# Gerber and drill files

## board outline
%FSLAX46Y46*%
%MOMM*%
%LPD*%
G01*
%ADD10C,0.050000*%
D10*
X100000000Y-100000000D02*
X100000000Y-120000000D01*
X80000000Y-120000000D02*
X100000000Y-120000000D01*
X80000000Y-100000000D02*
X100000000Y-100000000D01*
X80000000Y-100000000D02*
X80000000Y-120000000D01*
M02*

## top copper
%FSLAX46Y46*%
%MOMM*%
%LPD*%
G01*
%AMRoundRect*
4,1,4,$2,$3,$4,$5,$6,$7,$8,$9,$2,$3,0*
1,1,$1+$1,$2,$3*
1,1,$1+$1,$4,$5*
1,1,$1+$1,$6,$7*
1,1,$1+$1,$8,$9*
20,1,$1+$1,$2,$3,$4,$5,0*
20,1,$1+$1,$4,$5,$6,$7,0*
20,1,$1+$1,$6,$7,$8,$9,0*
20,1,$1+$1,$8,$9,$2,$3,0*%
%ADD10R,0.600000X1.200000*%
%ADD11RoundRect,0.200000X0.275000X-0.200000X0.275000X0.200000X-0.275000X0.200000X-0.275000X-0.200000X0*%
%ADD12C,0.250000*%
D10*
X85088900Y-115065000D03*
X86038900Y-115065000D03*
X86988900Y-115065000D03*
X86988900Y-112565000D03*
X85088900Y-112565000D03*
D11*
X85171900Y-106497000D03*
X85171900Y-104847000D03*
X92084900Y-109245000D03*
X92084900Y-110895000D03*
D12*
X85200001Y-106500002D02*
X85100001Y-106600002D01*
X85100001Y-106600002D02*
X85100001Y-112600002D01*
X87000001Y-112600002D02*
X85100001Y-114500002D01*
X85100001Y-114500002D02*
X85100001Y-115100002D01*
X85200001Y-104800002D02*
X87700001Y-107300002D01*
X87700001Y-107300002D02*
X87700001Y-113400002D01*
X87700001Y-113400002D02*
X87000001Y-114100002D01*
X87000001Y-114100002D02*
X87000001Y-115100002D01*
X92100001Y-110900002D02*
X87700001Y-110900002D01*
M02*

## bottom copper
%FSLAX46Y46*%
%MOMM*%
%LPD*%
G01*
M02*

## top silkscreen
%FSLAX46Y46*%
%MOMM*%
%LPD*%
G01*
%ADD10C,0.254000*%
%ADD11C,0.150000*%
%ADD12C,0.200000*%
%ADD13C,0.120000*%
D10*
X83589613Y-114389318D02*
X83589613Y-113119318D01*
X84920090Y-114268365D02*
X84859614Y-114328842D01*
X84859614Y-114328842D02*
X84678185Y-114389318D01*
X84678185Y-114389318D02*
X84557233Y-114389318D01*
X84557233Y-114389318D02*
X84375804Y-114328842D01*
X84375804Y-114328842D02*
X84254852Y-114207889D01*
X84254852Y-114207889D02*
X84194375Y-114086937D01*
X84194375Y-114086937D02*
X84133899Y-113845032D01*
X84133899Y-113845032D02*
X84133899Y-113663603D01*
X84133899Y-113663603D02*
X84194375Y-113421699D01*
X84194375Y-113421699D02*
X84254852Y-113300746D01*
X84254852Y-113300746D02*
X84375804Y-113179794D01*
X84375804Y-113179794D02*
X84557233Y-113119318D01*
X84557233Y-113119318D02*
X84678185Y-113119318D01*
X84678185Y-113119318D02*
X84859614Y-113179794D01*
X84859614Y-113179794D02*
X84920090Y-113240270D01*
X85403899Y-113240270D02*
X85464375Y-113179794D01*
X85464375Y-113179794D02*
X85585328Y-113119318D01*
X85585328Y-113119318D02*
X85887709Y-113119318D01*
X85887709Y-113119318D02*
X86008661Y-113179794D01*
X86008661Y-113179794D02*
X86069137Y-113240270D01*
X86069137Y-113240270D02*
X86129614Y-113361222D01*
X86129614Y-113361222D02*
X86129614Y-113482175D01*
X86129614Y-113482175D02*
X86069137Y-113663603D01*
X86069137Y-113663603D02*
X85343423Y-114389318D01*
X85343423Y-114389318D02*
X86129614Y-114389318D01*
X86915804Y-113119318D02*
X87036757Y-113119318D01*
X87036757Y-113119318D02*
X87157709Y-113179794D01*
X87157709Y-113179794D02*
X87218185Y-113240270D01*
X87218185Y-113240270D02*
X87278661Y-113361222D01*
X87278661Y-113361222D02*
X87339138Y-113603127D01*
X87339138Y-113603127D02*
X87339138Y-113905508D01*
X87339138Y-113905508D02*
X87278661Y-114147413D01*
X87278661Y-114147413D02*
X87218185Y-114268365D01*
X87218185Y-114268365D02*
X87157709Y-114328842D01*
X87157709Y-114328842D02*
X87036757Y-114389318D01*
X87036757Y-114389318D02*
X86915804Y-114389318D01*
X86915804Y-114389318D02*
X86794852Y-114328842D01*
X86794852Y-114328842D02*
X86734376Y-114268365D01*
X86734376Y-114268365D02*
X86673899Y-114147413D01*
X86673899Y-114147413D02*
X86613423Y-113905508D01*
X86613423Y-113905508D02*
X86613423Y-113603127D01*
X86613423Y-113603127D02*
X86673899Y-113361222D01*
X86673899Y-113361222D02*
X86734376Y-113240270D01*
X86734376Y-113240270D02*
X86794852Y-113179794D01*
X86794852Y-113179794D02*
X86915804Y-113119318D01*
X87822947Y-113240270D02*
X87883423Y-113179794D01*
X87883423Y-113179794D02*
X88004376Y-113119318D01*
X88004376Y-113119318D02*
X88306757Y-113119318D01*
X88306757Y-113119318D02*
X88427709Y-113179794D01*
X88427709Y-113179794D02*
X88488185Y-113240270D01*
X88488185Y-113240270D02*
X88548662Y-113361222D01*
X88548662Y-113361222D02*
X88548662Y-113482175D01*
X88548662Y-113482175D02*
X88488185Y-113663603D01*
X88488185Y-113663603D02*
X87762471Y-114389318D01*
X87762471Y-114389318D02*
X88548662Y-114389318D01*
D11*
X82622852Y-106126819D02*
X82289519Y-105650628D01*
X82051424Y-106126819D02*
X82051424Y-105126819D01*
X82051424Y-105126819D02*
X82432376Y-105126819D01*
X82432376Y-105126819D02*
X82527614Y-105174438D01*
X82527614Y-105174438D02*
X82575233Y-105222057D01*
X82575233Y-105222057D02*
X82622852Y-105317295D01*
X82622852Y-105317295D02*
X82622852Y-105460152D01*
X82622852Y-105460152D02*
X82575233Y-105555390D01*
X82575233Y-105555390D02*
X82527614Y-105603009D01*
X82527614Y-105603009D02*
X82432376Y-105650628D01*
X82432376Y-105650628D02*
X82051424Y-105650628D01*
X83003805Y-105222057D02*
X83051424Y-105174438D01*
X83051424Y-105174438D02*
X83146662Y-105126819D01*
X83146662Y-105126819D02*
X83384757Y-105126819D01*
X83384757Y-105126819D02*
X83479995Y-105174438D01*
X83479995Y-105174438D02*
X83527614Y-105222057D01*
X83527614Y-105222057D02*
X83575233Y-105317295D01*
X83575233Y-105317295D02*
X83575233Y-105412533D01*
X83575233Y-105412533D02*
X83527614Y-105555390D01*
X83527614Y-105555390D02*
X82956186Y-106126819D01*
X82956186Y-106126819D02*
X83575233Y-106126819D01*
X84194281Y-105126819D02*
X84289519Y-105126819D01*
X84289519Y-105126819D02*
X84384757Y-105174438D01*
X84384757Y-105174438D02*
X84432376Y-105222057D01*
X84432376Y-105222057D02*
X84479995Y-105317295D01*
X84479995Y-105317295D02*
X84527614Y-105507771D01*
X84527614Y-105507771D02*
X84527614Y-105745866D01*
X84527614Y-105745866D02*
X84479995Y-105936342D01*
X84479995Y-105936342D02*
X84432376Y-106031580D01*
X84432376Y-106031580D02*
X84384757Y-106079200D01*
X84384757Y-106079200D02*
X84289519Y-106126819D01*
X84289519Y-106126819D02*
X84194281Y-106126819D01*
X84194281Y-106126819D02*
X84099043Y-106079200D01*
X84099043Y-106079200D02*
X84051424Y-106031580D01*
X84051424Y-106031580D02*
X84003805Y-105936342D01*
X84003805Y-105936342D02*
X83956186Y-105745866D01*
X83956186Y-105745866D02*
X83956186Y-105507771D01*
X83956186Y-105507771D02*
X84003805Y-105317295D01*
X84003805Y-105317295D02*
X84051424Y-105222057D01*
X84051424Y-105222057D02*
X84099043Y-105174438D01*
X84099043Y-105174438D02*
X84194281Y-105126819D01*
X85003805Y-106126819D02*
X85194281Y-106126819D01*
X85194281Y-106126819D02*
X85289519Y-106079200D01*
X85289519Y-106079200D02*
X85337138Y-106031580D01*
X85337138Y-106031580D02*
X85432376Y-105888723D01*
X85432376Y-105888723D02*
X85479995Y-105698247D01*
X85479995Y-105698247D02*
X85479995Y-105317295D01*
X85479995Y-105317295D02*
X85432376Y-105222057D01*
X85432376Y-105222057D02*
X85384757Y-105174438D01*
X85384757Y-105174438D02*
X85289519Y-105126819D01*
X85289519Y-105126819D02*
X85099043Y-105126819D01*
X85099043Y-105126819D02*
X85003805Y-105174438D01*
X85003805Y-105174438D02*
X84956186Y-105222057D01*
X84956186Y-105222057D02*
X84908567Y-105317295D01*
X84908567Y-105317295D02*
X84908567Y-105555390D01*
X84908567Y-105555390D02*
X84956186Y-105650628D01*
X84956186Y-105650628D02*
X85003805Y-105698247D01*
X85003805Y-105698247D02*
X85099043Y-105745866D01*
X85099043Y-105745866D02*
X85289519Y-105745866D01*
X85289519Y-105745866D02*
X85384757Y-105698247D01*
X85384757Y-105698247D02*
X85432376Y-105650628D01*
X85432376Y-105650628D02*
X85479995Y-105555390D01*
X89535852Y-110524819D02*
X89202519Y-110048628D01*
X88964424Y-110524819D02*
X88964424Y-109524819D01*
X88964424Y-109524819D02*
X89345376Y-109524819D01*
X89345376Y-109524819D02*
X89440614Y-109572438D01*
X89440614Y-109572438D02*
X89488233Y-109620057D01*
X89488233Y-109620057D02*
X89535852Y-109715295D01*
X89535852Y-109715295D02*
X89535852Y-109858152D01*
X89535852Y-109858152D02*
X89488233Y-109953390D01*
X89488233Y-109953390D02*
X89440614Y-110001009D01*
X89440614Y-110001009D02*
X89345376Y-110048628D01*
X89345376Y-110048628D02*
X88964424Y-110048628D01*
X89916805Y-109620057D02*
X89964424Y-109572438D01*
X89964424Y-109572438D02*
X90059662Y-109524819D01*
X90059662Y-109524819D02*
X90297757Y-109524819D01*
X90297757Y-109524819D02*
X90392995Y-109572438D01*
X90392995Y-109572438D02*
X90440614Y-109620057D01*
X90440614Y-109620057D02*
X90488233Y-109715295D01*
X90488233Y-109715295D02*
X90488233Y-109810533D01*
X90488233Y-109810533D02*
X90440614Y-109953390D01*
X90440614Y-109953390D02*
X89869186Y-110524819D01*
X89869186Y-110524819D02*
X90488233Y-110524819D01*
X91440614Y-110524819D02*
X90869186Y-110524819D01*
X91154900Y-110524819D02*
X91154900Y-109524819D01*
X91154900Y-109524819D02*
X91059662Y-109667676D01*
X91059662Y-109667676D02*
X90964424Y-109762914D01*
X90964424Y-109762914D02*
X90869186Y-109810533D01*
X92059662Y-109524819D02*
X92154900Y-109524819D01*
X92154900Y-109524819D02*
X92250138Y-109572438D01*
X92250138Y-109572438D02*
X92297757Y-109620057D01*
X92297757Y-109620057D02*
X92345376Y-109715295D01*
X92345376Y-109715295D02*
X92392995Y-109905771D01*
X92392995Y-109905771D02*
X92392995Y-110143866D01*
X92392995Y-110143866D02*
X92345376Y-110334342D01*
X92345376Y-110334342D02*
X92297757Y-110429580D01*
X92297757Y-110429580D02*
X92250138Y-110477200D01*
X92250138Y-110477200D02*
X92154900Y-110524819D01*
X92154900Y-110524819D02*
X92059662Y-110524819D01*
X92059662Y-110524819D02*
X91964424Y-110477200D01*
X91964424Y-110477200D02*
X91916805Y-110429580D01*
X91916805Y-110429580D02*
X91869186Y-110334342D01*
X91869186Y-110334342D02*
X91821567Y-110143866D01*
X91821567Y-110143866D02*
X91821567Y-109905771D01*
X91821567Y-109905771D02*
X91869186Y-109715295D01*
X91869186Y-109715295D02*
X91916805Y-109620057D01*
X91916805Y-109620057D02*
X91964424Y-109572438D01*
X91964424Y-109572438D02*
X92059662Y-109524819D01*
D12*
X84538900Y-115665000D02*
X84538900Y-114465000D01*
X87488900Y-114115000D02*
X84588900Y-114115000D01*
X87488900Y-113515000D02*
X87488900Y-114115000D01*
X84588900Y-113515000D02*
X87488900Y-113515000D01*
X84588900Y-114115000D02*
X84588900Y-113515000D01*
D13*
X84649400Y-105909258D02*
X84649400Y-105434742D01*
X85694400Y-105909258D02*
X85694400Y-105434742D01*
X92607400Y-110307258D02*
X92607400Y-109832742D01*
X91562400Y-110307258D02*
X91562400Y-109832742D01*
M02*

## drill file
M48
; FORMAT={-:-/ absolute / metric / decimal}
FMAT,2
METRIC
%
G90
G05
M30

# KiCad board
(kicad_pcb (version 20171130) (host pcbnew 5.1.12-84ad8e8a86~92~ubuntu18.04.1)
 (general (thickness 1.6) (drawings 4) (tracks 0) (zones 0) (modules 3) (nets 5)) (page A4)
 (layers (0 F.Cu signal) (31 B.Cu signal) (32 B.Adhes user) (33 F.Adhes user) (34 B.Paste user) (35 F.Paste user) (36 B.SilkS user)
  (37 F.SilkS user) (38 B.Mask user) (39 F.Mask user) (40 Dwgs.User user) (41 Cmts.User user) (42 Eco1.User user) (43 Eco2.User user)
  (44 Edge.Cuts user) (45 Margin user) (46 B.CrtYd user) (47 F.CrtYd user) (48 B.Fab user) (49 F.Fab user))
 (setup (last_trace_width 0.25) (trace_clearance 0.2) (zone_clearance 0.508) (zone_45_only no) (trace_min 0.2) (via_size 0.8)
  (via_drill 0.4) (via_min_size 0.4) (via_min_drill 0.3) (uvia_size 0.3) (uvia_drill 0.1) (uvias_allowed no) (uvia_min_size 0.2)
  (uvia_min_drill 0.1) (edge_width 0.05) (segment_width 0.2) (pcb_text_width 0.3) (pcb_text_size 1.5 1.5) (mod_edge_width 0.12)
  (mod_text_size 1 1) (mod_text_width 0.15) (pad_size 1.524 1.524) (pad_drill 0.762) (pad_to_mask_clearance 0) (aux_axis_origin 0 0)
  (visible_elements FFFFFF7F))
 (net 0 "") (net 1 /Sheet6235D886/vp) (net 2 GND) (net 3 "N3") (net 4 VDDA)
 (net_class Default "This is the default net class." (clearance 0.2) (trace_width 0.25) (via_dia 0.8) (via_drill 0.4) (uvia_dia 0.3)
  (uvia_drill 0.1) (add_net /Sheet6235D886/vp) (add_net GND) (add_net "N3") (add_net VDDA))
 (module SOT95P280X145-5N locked (layer F.Cu) (at 86.038900 113.815000 90.000000)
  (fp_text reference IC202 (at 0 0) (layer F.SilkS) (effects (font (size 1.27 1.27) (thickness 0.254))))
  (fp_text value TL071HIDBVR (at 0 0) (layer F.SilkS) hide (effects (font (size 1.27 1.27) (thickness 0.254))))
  (fp_line (start -1.85 -1.5) (end -0.65 -1.5) (layer F.SilkS) (width 0.2))
  (fp_line (start -0.3 1.45) (end -0.3 -1.45) (layer F.SilkS) (width 0.2))
  (fp_line (start 0.3 1.45) (end -0.3 1.45) (layer F.SilkS) (width 0.2))
  (fp_line (start 0.3 -1.45) (end 0.3 1.45) (layer F.SilkS) (width 0.2))
  (fp_line (start -0.3 -1.45) (end 0.3 -1.45) (layer F.SilkS) (width 0.2))
  (pad 1 smd rect (at -1.25 -0.95 180.000000) (size 0.6 1.2) (layers F.Cu F.Mask F.Paste) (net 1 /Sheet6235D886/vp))
  (pad 2 smd rect (at -1.25 0 180.000000) (size 0.6 1.2) (layers F.Cu F.Mask F.Paste) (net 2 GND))
  (pad 3 smd rect (at -1.25 0.95 180.000000) (size 0.6 1.2) (layers F.Cu F.Mask F.Paste) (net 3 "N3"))
  (pad 4 smd rect (at 1.25 0.95 180.000000) (size 0.6 1.2) (layers F.Cu F.Mask F.Paste) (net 1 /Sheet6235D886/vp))
  (pad 5 smd rect (at 1.25 -0.95 180.000000) (size 0.6 1.2) (layers F.Cu F.Mask F.Paste) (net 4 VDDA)))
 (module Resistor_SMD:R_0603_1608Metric (layer F.Cu) (at 85.171900 105.672000 90.000000)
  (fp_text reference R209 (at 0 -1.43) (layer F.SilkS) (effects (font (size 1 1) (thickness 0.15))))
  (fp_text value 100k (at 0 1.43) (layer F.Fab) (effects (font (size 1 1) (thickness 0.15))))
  (fp_line (start -0.237258 -0.5225) (end 0.237258 -0.5225) (layer F.SilkS) (width 0.12))
  (fp_line (start -0.237258 0.5225) (end 0.237258 0.5225) (layer F.SilkS) (width 0.12))
  (pad 1 smd roundrect (at -0.825 0 90.000000) (size 0.8 0.95) (layers F.Cu F.Mask F.Paste) (roundrect_rratio 0.25) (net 4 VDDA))
  (pad 2 smd roundrect (at 0.825 0 90.000000) (size 0.8 0.95) (layers F.Cu F.Mask F.Paste) (roundrect_rratio 0.25) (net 3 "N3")))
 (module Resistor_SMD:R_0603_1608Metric (layer F.Cu) (at 92.084900 110.070000 90.000000)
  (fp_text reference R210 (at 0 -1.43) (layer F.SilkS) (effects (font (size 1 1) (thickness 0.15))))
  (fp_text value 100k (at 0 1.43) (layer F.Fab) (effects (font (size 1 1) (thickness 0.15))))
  (fp_line (start -0.237258 0.5225) (end 0.237258 0.5225) (layer F.SilkS) (width 0.12))
  (fp_line (start -0.237258 -0.5225) (end 0.237258 -0.5225) (layer F.SilkS) (width 0.12))
  (pad 2 smd roundrect (at 0.825 0 90.000000) (size 0.8 0.95) (layers F.Cu F.Mask F.Paste) (roundrect_rratio 0.25) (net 2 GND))
  (pad 1 smd roundrect (at -0.825 0 90.000000) (size 0.8 0.95) (layers F.Cu F.Mask F.Paste) (roundrect_rratio 0.25) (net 3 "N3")))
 (gr_line (start 100 100) (end 100 120) (layer Edge.Cuts) (width 0.05))
 (gr_line (start 80 120) (end 100 120) (layer Edge.Cuts) (width 0.05))
 (gr_line (start 80 100) (end 100 100) (layer Edge.Cuts) (width 0.05))
 (gr_line (start 80 100) (end 80 120) (layer Edge.Cuts) (width 0.05))
 (segment (start 85.200001 106.500002) (end 85.100001 106.600002) (width 0.250000) (layer F.Cu) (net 4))
 (segment (start 85.100001 106.600002) (end 85.100001 112.600002) (width 0.250000) (layer F.Cu) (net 4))
 (segment (start 87.000001 112.600002) (end 85.100001 114.500002) (width 0.250000) (layer F.Cu) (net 1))
 (segment (start 85.100001 114.500002) (end 85.100001 115.100002) (width 0.250000) (layer F.Cu) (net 1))
 (segment (start 85.200001 104.800002) (end 87.700001 107.300002) (width 0.250000) (layer F.Cu) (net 3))
 (segment (start 87.700001 107.300002) (end 87.700001 113.400002) (width 0.250000) (layer F.Cu) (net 3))
 (segment (start 87.700001 113.400002) (end 87.000001 114.100002) (width 0.250000) (layer F.Cu) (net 3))
 (segment (start 87.000001 114.100002) (end 87.000001 115.100002) (width 0.250000) (layer F.Cu) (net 3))
 (segment (start 92.100001 110.900002) (end 87.700001 110.900002) (width 0.250000) (layer F.Cu) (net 3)))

